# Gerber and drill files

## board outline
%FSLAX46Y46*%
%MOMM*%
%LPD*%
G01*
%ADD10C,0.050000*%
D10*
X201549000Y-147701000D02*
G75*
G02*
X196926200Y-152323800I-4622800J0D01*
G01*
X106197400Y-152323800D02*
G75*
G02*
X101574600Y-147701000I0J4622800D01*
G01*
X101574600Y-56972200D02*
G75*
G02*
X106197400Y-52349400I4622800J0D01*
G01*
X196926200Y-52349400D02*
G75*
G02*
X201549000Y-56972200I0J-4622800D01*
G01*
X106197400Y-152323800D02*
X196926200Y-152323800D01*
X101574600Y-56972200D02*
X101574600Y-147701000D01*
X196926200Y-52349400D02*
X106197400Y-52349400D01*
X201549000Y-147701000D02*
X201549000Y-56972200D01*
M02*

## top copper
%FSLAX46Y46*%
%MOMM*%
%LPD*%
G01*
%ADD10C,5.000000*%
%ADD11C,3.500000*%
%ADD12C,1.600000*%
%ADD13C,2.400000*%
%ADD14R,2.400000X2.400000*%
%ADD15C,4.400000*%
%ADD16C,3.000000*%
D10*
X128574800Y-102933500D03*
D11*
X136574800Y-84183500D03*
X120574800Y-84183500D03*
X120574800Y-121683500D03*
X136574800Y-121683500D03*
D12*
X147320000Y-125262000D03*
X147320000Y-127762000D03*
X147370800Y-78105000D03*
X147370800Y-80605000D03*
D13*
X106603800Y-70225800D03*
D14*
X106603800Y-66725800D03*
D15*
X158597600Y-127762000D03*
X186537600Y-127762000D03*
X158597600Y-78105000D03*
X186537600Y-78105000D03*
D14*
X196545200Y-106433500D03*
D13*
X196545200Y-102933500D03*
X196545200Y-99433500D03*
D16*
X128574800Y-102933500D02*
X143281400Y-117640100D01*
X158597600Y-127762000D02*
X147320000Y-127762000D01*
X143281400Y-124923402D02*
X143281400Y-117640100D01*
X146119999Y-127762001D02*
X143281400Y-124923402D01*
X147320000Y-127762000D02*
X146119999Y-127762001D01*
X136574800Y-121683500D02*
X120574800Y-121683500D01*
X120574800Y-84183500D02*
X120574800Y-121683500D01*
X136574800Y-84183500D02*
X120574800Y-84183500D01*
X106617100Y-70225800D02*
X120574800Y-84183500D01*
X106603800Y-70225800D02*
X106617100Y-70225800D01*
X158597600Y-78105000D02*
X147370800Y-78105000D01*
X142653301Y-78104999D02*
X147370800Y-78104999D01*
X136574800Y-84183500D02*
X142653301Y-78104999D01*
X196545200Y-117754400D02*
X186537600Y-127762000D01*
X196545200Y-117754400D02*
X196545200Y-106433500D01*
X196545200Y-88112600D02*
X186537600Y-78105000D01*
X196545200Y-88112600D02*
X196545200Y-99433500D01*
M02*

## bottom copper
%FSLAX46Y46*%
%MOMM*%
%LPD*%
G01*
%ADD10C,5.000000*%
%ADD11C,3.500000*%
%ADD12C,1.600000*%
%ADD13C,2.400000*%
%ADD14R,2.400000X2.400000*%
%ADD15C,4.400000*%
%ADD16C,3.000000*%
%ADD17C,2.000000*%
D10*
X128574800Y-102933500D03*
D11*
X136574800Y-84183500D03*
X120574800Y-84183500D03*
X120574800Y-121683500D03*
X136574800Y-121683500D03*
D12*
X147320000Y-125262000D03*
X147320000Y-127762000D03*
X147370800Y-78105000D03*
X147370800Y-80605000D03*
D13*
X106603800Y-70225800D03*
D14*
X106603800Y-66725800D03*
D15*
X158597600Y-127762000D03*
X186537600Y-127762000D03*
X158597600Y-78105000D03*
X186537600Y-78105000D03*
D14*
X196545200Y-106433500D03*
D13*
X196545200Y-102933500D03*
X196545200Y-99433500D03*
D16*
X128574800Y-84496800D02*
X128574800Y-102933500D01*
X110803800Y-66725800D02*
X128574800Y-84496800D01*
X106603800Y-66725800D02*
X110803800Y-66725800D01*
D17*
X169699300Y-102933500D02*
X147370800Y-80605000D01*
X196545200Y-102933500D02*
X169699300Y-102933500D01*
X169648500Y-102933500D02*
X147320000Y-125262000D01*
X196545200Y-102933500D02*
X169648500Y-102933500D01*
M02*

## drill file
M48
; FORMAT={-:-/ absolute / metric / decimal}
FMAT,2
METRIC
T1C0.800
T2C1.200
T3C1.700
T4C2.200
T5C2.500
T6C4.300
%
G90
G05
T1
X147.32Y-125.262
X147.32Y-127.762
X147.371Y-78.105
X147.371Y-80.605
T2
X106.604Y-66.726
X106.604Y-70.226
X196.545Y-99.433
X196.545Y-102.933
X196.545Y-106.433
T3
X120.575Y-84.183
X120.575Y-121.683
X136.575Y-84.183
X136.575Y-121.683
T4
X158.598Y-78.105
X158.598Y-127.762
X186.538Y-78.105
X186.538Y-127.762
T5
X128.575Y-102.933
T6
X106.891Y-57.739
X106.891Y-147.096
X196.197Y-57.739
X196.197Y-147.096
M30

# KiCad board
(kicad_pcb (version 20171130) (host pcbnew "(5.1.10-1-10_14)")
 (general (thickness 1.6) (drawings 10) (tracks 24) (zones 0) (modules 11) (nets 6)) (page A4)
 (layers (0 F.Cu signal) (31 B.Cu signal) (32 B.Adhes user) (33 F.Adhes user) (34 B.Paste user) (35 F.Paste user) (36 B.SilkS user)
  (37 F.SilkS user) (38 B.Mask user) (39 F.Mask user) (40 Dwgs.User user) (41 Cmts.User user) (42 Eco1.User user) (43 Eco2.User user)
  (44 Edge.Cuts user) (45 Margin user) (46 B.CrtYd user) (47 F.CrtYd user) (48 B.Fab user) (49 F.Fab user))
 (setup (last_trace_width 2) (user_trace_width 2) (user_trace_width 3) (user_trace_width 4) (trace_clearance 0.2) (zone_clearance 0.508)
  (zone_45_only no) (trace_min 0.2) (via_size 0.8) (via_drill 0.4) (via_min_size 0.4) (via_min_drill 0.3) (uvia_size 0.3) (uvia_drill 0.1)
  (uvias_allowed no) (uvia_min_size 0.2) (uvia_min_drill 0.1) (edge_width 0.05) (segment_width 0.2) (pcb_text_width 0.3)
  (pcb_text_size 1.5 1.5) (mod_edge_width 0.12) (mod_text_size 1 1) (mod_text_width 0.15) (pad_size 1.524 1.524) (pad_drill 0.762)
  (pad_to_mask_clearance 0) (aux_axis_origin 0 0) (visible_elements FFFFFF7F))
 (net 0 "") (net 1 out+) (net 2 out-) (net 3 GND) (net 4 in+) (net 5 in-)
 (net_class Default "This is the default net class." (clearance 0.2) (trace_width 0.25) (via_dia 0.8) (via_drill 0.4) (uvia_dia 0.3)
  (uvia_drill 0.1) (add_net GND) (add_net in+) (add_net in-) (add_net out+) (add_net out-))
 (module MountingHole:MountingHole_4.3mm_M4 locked (layer F.Cu) (at 196.197 147.0962)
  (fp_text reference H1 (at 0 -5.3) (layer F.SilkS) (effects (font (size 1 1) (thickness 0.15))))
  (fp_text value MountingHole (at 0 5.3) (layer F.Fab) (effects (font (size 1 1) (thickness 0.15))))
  (pad 1 np_thru_hole circle (at 0 0) (size 4.3 4.3) (drill 4.3) (layers *.Cu *.Mask)))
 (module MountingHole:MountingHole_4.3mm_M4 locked (layer F.Cu) (at 196.197 57.739)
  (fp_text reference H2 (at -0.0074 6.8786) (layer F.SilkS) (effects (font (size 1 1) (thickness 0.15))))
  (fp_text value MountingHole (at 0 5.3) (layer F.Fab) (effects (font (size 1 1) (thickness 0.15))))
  (pad 1 np_thru_hole circle (at 0 0) (size 4.3 4.3) (drill 4.3) (layers *.Cu *.Mask)))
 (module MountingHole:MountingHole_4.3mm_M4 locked (layer F.Cu) (at 106.8906 147.0962)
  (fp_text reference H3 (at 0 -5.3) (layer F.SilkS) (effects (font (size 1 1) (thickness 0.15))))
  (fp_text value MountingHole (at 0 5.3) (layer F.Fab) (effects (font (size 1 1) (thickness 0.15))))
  (pad 1 np_thru_hole circle (at 0 0) (size 4.3 4.3) (drill 4.3) (layers *.Cu *.Mask)))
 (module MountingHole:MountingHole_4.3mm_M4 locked (layer F.Cu) (at 106.8906 57.739)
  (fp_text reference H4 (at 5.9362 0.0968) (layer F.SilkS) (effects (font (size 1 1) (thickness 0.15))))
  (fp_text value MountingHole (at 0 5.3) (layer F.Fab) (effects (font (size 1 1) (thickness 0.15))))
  (pad 1 np_thru_hole circle (at 0 0) (size 4.3 4.3) (drill 4.3) (layers *.Cu *.Mask)))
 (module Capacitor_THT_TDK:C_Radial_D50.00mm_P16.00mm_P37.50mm (layer F.Cu) (at 128.5748 102.9335)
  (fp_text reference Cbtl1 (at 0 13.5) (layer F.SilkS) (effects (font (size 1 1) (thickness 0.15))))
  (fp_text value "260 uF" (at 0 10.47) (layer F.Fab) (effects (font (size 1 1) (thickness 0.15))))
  (pad 2 thru_hole circle (at 0 0) (size 5 5) (drill 2.5) (layers *.Cu *.Mask) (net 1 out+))
  (pad 1 thru_hole circle (at 8 -18.75) (size 3.5 3.5) (drill 1.7) (layers *.Cu *.Mask) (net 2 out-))
  (pad 1 thru_hole circle (at -8 -18.75) (size 3.5 3.5) (drill 1.7) (layers *.Cu *.Mask) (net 2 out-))
  (pad 1 thru_hole circle (at -8 18.75) (size 3.5 3.5) (drill 1.7) (layers *.Cu *.Mask) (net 2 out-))
  (pad 1 thru_hole circle (at 8 18.75) (size 3.5 3.5) (drill 1.7) (layers *.Cu *.Mask) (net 2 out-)))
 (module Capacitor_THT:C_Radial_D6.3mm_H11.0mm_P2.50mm (layer F.Cu) (at 147.32 127.762 90)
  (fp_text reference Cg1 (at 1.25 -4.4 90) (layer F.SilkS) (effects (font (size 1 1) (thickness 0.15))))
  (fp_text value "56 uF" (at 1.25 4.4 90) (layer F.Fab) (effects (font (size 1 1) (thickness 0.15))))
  (pad 2 thru_hole circle (at 2.5 0 90) (size 1.6 1.6) (drill 0.8) (layers *.Cu *.Mask) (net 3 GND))
  (pad 1 thru_hole circle (at 0 0 90) (size 1.6 1.6) (drill 0.8) (layers *.Cu *.Mask) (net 1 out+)))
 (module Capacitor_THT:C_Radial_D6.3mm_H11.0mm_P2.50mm (layer F.Cu) (at 147.3708 78.105 270)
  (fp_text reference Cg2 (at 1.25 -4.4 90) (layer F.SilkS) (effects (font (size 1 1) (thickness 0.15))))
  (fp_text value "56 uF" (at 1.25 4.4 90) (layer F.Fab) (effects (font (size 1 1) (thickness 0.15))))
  (pad 1 thru_hole circle (at 0 0 270) (size 1.6 1.6) (drill 0.8) (layers *.Cu *.Mask) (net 2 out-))
  (pad 2 thru_hole circle (at 2.5 0 270) (size 1.6 1.6) (drill 0.8) (layers *.Cu *.Mask) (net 3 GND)))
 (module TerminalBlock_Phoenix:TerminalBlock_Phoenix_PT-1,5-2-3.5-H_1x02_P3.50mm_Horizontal (layer F.Cu) (at 106.6038 66.7258 270)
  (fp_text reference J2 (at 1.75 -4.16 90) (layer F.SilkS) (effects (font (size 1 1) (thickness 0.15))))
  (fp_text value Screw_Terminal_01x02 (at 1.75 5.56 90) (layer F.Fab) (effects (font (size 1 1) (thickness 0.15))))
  (pad 2 thru_hole circle (at 3.5 0 270) (size 2.4 2.4) (drill 1.2) (layers *.Cu *.Mask) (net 2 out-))
  (pad 1 thru_hole rect (at 0 0 270) (size 2.4 2.4) (drill 1.2) (layers *.Cu *.Mask) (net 1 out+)))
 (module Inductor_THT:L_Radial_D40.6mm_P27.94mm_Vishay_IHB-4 (layer F.Cu) (at 158.5976 127.762)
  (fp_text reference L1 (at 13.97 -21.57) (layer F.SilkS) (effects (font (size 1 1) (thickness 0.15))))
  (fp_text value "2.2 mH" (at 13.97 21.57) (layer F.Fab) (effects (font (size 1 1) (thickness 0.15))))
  (pad 1 thru_hole circle (at 0 0) (size 4.4 4.4) (drill 2.2) (layers *.Cu *.Mask) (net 1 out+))
  (pad 2 thru_hole circle (at 27.94 0) (size 4.4 4.4) (drill 2.2) (layers *.Cu *.Mask) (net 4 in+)))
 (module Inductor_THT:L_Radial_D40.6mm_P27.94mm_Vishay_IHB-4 (layer F.Cu) (at 186.5376 78.105 180)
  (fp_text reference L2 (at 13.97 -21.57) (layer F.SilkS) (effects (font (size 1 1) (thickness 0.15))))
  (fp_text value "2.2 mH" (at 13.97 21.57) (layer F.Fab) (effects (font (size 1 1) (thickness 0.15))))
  (pad 2 thru_hole circle (at 27.94 0 180) (size 4.4 4.4) (drill 2.2) (layers *.Cu *.Mask) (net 2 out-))
  (pad 1 thru_hole circle (at 0 0 180) (size 4.4 4.4) (drill 2.2) (layers *.Cu *.Mask) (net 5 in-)))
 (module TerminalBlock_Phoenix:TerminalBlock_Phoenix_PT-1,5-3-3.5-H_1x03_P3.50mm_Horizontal (layer F.Cu) (at 196.5452 106.4335 90)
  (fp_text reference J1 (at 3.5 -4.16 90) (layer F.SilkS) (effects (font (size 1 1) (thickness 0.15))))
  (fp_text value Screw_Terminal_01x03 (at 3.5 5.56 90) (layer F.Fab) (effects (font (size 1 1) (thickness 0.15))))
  (pad 1 thru_hole rect (at 0 0 90) (size 2.4 2.4) (drill 1.2) (layers *.Cu *.Mask) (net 4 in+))
  (pad 2 thru_hole circle (at 3.5 0 90) (size 2.4 2.4) (drill 1.2) (layers *.Cu *.Mask) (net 3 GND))
  (pad 3 thru_hole circle (at 7 0 90) (size 2.4 2.4) (drill 1.2) (layers *.Cu *.Mask) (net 5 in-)))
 (gr_arc (start 196.9262 147.701) (end 196.9262 152.3238) (angle -90) (layer Edge.Cuts) (width 0.05))
 (gr_arc (start 106.1974 147.701) (end 101.5746 147.701) (angle -90) (layer Edge.Cuts) (width 0.05))
 (gr_arc (start 106.1974 56.9722) (end 106.1974 52.3494) (angle -90) (layer Edge.Cuts) (width 0.05))
 (gr_arc (start 196.9262 56.9722) (end 201.549 56.9722) (angle -90) (layer Edge.Cuts) (width 0.05))
 (gr_line (start 106.1974 152.3238) (end 196.9262 152.3238) (layer Edge.Cuts) (width 0.05))
 (gr_line (start 101.5746 56.9722) (end 101.5746 147.701) (layer Edge.Cuts) (width 0.05))
 (gr_line (start 196.9262 52.3494) (end 106.1974 52.3494) (layer Edge.Cuts) (width 0.05))
 (gr_line (start 201.549 147.701) (end 201.549 56.9722) (layer Edge.Cuts) (width 0.05))
 (segment (start 128.5748 84.4968) (end 128.5748 102.9335) (width 3) (layer B.Cu) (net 1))
 (segment (start 110.8038 66.7258) (end 128.5748 84.4968) (width 3) (layer B.Cu) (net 1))
 (segment (start 106.6038 66.7258) (end 110.8038 66.7258) (width 3) (layer B.Cu) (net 1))
 (segment (start 128.5748 102.9335) (end 143.2814 117.6401) (width 3) (layer F.Cu) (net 1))
 (segment (start 158.5976 127.762) (end 147.32 127.762) (width 3) (layer F.Cu) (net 1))
 (segment (start 143.2814 124.923402) (end 143.2814 117.6401) (width 3) (layer F.Cu) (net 1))
 (segment (start 146.119999 127.762001) (end 143.2814 124.923402) (width 3) (layer F.Cu) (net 1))
 (segment (start 147.32 127.762) (end 146.119999 127.762001) (width 3) (layer F.Cu) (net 1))
 (segment (start 136.5748 121.6835) (end 120.5748 121.6835) (width 3) (layer F.Cu) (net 2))
 (segment (start 120.5748 84.1835) (end 120.5748 121.6835) (width 3) (layer F.Cu) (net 2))
 (segment (start 136.5748 84.1835) (end 120.5748 84.1835) (width 3) (layer F.Cu) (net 2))
 (segment (start 106.6171 70.2258) (end 120.5748 84.1835) (width 3) (layer F.Cu) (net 2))
 (segment (start 106.6038 70.2258) (end 106.6171 70.2258) (width 3) (layer F.Cu) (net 2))
 (segment (start 158.5976 78.105) (end 147.3708 78.105) (width 3) (layer F.Cu) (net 2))
 (segment (start 142.653301 78.104999) (end 147.3708 78.104999) (width 3) (layer F.Cu) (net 2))
 (segment (start 136.5748 84.1835) (end 142.653301 78.104999) (width 3) (layer F.Cu) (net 2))
 (segment (start 169.6993 102.9335) (end 147.3708 80.605) (width 2) (layer B.Cu) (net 3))
 (segment (start 196.5452 102.9335) (end 169.6993 102.9335) (width 2) (layer B.Cu) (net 3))
 (segment (start 169.6485 102.9335) (end 147.32 125.262) (width 2) (layer B.Cu) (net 3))
 (segment (start 196.5452 102.9335) (end 169.6485 102.9335) (width 2) (layer B.Cu) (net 3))
 (segment (start 196.5452 117.7544) (end 186.5376 127.762) (width 3) (layer F.Cu) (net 4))
 (segment (start 196.5452 117.7544) (end 196.5452 106.4335) (width 3) (layer F.Cu) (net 4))
 (segment (start 196.5452 88.1126) (end 186.5376 78.105) (width 3) (layer F.Cu) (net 5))
 (segment (start 196.5452 88.1126) (end 196.5452 99.4335) (width 3) (layer F.Cu) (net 5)))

